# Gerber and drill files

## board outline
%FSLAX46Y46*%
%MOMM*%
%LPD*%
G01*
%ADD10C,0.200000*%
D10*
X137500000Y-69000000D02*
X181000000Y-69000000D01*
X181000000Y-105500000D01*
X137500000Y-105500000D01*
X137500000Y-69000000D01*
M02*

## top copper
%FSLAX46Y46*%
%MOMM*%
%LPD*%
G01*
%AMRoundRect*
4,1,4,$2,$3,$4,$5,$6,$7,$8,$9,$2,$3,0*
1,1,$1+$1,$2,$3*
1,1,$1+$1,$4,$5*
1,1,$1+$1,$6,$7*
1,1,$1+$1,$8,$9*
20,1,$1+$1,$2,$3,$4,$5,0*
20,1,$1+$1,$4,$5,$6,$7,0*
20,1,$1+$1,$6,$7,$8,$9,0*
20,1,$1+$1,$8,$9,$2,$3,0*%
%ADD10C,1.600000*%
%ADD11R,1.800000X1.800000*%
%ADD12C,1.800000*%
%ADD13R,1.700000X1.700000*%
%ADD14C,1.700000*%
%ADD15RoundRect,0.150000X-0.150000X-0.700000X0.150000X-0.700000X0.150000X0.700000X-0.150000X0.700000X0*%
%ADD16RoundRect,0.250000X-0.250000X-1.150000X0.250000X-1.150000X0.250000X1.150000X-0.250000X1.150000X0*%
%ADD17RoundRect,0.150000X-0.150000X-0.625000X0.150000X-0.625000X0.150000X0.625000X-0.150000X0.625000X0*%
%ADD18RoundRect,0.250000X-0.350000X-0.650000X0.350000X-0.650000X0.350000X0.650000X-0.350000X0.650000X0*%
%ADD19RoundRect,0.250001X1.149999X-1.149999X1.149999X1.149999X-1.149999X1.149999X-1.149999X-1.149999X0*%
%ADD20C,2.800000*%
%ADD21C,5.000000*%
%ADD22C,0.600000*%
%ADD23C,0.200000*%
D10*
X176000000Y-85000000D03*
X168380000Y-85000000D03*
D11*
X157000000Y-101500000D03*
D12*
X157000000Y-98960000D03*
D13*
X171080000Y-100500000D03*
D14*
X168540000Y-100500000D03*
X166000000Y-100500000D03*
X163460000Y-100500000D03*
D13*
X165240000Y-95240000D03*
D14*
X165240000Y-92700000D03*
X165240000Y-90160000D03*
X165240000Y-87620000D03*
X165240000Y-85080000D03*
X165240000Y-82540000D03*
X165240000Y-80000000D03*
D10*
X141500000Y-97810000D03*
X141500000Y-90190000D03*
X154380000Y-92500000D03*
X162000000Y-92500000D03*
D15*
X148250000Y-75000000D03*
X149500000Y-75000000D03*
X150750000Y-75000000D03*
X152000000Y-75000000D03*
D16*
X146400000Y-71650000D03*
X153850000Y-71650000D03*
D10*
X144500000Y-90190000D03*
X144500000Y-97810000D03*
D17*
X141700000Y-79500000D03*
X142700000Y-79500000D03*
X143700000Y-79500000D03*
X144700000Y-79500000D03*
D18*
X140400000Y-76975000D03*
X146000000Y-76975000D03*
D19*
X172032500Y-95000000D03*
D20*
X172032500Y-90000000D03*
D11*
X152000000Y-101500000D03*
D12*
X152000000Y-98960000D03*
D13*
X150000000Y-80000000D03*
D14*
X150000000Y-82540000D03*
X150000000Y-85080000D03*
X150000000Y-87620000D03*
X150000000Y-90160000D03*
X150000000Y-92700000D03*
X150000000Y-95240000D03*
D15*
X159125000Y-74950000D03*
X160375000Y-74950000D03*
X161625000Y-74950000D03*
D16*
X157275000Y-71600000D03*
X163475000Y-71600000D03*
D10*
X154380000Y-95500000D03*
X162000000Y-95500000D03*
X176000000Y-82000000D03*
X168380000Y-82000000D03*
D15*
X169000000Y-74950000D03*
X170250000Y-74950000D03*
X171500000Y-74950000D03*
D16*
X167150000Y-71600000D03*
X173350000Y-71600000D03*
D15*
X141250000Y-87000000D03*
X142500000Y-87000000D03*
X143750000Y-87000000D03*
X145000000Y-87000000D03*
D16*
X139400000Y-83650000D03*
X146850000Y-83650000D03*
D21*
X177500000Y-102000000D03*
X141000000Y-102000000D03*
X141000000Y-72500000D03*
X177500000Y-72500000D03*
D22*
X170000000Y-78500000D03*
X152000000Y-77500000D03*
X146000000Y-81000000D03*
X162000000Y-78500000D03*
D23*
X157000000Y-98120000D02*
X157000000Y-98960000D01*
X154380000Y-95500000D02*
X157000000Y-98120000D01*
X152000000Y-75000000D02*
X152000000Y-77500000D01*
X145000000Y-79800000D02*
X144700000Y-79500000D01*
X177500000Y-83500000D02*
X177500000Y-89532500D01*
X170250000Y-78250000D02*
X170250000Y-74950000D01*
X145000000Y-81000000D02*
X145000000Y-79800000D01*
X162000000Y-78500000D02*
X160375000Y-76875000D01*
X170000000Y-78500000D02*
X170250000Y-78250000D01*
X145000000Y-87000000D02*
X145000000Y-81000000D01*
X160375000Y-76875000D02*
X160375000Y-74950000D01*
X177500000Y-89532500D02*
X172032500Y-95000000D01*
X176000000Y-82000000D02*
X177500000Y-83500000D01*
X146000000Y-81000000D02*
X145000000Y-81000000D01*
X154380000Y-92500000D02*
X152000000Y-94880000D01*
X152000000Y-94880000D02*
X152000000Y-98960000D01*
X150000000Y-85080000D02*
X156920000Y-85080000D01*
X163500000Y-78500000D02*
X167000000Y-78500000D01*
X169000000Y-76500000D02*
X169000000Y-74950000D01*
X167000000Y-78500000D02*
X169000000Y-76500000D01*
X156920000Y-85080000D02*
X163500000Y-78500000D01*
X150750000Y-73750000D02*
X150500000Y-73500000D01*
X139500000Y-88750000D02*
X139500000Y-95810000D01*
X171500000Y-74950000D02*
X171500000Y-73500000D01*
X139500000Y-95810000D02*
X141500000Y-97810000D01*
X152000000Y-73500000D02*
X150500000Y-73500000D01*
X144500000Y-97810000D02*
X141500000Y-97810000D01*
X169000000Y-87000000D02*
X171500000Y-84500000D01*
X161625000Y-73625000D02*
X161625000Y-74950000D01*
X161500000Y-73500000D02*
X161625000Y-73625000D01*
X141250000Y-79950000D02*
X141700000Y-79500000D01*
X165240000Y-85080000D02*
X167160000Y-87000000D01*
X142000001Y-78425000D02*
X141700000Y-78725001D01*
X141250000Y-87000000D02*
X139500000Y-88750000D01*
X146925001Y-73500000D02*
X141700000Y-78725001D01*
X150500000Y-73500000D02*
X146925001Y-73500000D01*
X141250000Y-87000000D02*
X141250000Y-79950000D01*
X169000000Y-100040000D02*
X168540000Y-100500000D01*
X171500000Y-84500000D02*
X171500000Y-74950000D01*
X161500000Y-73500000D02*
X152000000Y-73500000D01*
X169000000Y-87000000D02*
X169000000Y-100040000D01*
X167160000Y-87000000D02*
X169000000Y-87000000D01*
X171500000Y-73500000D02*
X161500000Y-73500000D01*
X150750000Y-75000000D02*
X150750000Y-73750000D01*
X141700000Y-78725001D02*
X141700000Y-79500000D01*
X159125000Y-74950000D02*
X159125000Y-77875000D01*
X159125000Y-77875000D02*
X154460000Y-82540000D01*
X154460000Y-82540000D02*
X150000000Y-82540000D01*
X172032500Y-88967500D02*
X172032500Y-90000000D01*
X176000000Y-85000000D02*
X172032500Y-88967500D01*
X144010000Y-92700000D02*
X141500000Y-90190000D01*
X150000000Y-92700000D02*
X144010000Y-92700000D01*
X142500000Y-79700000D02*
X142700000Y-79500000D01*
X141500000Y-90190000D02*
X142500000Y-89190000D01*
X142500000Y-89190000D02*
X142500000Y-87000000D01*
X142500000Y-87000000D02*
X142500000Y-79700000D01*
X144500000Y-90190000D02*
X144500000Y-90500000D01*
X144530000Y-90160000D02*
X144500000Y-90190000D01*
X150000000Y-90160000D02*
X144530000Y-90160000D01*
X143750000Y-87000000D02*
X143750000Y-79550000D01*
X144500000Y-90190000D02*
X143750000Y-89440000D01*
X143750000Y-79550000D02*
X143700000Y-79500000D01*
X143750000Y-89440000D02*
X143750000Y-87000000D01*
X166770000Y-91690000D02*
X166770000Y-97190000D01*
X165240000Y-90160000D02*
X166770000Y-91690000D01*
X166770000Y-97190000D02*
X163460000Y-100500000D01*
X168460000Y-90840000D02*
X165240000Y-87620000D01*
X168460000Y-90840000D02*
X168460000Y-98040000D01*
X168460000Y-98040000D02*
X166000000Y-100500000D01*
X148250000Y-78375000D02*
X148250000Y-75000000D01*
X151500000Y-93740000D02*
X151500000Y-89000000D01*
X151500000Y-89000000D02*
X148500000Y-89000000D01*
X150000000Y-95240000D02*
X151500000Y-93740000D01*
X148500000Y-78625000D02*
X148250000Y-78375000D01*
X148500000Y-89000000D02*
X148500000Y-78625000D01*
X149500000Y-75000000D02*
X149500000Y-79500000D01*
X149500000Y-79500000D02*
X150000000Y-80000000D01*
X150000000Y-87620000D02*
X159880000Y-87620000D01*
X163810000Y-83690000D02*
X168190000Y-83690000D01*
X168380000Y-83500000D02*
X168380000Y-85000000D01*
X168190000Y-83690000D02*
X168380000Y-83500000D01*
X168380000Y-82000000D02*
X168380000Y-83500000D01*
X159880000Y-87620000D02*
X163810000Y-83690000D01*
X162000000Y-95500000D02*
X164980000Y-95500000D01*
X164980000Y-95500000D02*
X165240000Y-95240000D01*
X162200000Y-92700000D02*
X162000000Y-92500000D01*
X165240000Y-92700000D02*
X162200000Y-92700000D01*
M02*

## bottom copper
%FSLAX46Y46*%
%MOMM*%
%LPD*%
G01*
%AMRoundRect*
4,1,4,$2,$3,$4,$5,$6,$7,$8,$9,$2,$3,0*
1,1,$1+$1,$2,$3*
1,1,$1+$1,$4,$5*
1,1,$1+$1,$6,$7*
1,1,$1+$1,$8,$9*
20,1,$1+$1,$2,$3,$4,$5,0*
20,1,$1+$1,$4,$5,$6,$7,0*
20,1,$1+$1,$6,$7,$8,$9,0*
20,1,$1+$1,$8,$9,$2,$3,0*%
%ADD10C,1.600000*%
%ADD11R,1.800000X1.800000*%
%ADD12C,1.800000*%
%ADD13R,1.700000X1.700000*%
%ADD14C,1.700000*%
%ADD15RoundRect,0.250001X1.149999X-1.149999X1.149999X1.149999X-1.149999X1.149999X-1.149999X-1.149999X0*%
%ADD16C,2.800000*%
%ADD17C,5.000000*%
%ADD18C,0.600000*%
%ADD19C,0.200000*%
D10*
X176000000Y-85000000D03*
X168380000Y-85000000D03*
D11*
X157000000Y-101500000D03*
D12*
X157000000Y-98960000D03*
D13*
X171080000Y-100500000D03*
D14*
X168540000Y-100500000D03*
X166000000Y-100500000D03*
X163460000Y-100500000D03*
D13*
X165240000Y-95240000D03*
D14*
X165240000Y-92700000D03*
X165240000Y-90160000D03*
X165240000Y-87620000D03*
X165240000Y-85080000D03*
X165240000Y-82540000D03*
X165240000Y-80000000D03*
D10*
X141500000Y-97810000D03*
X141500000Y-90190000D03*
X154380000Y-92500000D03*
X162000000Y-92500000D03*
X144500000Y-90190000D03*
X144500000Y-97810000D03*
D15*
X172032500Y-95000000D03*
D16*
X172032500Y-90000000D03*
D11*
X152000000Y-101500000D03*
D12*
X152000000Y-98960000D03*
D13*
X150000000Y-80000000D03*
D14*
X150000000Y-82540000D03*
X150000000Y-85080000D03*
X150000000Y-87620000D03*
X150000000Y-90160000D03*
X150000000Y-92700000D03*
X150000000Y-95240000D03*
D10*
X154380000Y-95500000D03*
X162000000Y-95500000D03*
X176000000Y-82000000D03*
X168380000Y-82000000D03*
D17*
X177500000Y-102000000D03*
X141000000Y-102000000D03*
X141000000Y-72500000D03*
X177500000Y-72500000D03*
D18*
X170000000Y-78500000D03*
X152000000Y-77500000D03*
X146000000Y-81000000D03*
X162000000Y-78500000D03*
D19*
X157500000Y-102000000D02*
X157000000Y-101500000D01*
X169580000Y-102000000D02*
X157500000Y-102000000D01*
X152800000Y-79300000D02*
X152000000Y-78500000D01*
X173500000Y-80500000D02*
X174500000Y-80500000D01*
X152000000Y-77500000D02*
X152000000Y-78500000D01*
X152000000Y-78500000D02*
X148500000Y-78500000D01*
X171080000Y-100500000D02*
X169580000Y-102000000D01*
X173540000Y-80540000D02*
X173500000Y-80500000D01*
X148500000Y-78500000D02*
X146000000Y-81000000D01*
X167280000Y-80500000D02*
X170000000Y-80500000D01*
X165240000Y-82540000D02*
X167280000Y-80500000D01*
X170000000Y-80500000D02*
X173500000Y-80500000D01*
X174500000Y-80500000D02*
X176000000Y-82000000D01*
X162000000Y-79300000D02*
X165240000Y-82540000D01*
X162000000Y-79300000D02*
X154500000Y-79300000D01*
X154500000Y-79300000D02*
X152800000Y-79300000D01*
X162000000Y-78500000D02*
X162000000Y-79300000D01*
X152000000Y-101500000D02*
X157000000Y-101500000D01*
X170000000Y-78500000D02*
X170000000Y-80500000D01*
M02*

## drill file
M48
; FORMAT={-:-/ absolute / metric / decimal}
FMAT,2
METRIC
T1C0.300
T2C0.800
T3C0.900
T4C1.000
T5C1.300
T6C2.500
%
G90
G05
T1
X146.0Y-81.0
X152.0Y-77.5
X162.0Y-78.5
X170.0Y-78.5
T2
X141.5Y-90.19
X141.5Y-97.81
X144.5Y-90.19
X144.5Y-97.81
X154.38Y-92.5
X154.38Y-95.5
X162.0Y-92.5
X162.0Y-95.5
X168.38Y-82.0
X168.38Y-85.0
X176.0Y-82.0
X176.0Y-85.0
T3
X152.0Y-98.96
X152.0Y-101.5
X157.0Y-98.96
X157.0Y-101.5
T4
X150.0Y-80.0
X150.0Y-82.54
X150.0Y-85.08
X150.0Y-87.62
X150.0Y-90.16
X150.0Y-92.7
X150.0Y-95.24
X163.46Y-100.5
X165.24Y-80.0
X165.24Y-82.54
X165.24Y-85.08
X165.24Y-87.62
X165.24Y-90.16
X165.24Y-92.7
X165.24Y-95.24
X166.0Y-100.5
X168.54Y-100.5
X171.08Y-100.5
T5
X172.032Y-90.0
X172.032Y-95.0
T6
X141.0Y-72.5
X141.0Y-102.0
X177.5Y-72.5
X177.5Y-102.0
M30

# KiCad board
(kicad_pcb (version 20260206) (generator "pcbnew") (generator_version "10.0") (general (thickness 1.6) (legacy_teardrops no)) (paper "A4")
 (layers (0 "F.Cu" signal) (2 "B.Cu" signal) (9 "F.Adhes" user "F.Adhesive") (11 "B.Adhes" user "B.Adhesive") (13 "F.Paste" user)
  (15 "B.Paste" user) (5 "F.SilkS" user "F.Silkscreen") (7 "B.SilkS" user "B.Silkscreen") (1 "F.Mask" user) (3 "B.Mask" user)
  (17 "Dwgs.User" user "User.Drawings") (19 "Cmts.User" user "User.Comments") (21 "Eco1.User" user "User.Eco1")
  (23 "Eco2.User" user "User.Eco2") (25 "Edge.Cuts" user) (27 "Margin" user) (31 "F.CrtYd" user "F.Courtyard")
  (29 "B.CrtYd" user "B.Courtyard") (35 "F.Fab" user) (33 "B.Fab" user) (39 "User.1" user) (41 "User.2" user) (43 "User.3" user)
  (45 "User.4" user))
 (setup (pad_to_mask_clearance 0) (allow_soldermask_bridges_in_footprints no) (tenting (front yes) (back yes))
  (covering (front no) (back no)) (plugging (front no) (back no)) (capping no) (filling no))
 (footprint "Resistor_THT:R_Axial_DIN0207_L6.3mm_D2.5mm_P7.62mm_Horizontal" (layer "F.Cu") (at 176 85 180)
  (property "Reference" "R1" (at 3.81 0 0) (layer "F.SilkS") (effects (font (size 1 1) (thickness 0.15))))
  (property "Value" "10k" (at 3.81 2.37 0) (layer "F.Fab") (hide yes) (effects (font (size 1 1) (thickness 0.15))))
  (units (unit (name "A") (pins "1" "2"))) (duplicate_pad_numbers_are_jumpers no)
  (pad "1" thru_hole circle (at 0 0 180) (size 1.6 1.6) (drill 0.8) (layers "*.Cu" "*.Mask") (remove_unused_layers no)
   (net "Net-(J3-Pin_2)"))
  (pad "2" thru_hole circle (at 7.62 0 180) (size 1.6 1.6) (drill 0.8) (layers "*.Cu" "*.Mask") (remove_unused_layers no)
   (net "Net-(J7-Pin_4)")))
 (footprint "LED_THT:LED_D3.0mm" (layer "F.Cu") (at 157 101.5 90)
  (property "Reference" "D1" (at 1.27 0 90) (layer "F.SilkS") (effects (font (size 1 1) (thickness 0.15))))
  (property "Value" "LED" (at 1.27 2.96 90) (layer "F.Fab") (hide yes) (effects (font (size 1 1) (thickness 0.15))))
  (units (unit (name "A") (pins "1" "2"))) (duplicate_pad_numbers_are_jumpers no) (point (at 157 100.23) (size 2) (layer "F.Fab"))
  (pad "1" thru_hole rect (at 0 0 90) (size 1.8 1.8) (drill 0.9) (layers "*.Cu" "*.Mask") (remove_unused_layers no) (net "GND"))
  (pad "2" thru_hole circle (at 2.54 0 90) (size 1.8 1.8) (drill 0.9) (layers "*.Cu" "*.Mask") (remove_unused_layers no) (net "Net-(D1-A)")))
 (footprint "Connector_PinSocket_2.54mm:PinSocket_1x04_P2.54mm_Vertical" (layer "F.Cu") (at 171.08 100.5 -90)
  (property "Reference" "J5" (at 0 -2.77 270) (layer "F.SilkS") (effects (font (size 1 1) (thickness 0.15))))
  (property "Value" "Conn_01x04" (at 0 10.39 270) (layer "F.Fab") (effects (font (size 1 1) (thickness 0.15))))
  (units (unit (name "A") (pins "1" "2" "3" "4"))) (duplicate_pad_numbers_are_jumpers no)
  (pad "1" thru_hole rect (at 0 0 270) (size 1.7 1.7) (drill 1) (layers "*.Cu" "*.Mask") (remove_unused_layers no) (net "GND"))
  (pad "2" thru_hole circle (at 0 2.54 270) (size 1.7 1.7) (drill 1) (layers "*.Cu" "*.Mask") (remove_unused_layers no)
   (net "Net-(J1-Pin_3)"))
  (pad "3" thru_hole circle (at 0 5.08 270) (size 1.7 1.7) (drill 1) (layers "*.Cu" "*.Mask") (remove_unused_layers no)
   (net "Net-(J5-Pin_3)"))
  (pad "4" thru_hole circle (at 0 7.62 270) (size 1.7 1.7) (drill 1) (layers "*.Cu" "*.Mask") (remove_unused_layers no)
   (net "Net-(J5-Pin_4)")))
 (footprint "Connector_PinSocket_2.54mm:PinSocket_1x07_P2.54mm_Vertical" (layer "F.Cu") (at 165.24 95.24 180)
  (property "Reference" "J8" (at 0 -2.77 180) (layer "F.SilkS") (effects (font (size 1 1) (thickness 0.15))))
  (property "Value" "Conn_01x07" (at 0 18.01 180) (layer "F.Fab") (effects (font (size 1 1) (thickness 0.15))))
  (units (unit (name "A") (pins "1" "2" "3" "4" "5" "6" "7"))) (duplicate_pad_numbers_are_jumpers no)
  (pad "1" thru_hole rect (at 0 0 180) (size 1.7 1.7) (drill 1) (layers "*.Cu" "*.Mask") (remove_unused_layers no) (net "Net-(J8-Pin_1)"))
  (pad "2" thru_hole circle (at 0 2.54 180) (size 1.7 1.7) (drill 1) (layers "*.Cu" "*.Mask") (remove_unused_layers no)
   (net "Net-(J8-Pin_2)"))
  (pad "3" thru_hole circle (at 0 5.08 180) (size 1.7 1.7) (drill 1) (layers "*.Cu" "*.Mask") (remove_unused_layers no)
   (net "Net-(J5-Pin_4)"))
  (pad "4" thru_hole circle (at 0 7.62 180) (size 1.7 1.7) (drill 1) (layers "*.Cu" "*.Mask") (remove_unused_layers no)
   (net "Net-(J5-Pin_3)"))
  (pad "5" thru_hole circle (at 0 10.16 180) (size 1.7 1.7) (drill 1) (layers "*.Cu" "*.Mask") (remove_unused_layers no)
   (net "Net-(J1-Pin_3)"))
  (pad "6" thru_hole circle (at 0 12.7 180) (size 1.7 1.7) (drill 1) (layers "*.Cu" "*.Mask") (remove_unused_layers no) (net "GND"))
  (pad "7" thru_hole circle (at 0 15.24 180) (size 1.7 1.7) (drill 1) (layers "*.Cu" "*.Mask") (remove_unused_layers no)
   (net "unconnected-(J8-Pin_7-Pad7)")))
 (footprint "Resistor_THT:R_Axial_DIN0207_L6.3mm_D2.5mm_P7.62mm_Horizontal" (layer "F.Cu") (at 141.5 97.81 90)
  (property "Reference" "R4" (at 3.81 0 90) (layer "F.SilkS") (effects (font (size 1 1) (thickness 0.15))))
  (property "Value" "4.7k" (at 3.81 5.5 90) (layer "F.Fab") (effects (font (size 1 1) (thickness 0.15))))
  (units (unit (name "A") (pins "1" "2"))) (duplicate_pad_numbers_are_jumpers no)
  (pad "1" thru_hole circle (at 0 0 90) (size 1.6 1.6) (drill 0.8) (layers "*.Cu" "*.Mask") (remove_unused_layers no) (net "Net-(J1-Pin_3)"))
  (pad "2" thru_hole circle (at 7.62 0 90) (size 1.6 1.6) (drill 0.8) (layers "*.Cu" "*.Mask") (remove_unused_layers no)
   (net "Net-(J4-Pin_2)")))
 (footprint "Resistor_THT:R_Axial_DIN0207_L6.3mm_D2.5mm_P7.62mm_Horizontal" (layer "F.Cu") (at 154.38 92.5)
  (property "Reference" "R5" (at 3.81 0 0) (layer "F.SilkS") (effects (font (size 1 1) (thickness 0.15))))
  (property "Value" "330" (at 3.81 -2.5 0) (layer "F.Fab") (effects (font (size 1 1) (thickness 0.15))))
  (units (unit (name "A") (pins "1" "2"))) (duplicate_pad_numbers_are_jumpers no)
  (pad "1" thru_hole circle (at 0 0) (size 1.6 1.6) (drill 0.8) (layers "*.Cu" "*.Mask") (remove_unused_layers no) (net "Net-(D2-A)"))
  (pad "2" thru_hole circle (at 7.62 0) (size 1.6 1.6) (drill 0.8) (layers "*.Cu" "*.Mask") (remove_unused_layers no) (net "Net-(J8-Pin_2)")))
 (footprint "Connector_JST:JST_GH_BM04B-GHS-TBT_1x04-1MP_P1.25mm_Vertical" (layer "F.Cu") (at 150.125 73.05)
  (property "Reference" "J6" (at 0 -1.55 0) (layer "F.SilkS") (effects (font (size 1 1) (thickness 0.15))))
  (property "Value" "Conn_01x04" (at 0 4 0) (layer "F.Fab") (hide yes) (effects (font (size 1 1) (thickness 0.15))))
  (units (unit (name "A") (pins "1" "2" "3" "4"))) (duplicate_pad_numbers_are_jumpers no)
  (pad "1" smd roundrect (at -1.875 1.95) (size 0.6 1.7) (layers "F.Cu" "F.Mask" "F.Paste") (roundrect_rratio 0.25) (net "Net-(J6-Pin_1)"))
  (pad "2" smd roundrect (at -0.625 1.95) (size 0.6 1.7) (layers "F.Cu" "F.Mask" "F.Paste") (roundrect_rratio 0.25) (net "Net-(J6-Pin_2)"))
  (pad "3" smd roundrect (at 0.625 1.95) (size 0.6 1.7) (layers "F.Cu" "F.Mask" "F.Paste") (roundrect_rratio 0.25) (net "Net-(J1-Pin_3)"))
  (pad "4" smd roundrect (at 1.875 1.95) (size 0.6 1.7) (layers "F.Cu" "F.Mask" "F.Paste") (roundrect_rratio 0.25) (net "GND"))
  (pad "MP" smd roundrect (at -3.725 -1.4) (size 1 2.8) (layers "F.Cu" "F.Mask" "F.Paste") (roundrect_rratio 0.25))
  (pad "MP" smd roundrect (at 3.725 -1.4) (size 1 2.8) (layers "F.Cu" "F.Mask" "F.Paste") (roundrect_rratio 0.25)))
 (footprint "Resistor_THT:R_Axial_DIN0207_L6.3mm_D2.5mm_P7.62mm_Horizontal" (layer "F.Cu") (at 144.5 90.19 -90)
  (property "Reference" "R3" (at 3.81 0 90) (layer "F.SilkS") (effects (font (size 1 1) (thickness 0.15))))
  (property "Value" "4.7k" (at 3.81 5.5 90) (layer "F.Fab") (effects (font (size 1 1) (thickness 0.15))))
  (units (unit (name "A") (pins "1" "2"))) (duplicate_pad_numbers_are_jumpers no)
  (pad "1" thru_hole circle (at 0 0 270) (size 1.6 1.6) (drill 0.8) (layers "*.Cu" "*.Mask") (remove_unused_layers no)
   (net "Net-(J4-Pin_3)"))
  (pad "2" thru_hole circle (at 7.62 0 270) (size 1.6 1.6) (drill 0.8) (layers "*.Cu" "*.Mask") (remove_unused_layers no)
   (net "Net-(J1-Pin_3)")))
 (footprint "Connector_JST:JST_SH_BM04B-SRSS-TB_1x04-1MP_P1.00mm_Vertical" (layer "F.Cu") (at 143.2 78.175)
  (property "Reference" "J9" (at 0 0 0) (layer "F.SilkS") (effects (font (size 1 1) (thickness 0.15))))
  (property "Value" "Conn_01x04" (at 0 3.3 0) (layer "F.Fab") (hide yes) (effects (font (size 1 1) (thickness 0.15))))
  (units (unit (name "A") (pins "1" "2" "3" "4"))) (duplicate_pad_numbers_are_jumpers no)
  (pad "1" smd roundrect (at -1.5 1.325) (size 0.6 1.55) (layers "F.Cu" "F.Mask" "F.Paste") (roundrect_rratio 0.25) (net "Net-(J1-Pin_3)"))
  (pad "2" smd roundrect (at -0.5 1.325) (size 0.6 1.55) (layers "F.Cu" "F.Mask" "F.Paste") (roundrect_rratio 0.25) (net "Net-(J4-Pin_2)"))
  (pad "3" smd roundrect (at 0.5 1.325) (size 0.6 1.55) (layers "F.Cu" "F.Mask" "F.Paste") (roundrect_rratio 0.25) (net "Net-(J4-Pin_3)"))
  (pad "4" smd roundrect (at 1.5 1.325) (size 0.6 1.55) (layers "F.Cu" "F.Mask" "F.Paste") (roundrect_rratio 0.25) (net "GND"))
  (pad "MP" smd roundrect (at -2.8 -1.2) (size 1.2 1.8) (layers "F.Cu" "F.Mask" "F.Paste") (roundrect_rratio 0.208333))
  (pad "MP" smd roundrect (at 2.8 -1.2) (size 1.2 1.8) (layers "F.Cu" "F.Mask" "F.Paste") (roundrect_rratio 0.208333)))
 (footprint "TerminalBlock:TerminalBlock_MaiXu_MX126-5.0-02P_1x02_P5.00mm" (layer "F.Cu") (at 172.0325 95 90)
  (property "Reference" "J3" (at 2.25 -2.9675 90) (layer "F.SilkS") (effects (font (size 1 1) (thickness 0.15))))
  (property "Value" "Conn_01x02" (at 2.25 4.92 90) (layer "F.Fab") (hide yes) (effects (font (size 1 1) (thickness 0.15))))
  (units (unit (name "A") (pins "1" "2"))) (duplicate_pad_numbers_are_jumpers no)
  (pad "1" thru_hole roundrect (at 0 0 90) (size 2.8 2.8) (drill 1.3) (layers "*.Cu" "*.Mask") (remove_unused_layers no)
   (roundrect_rratio 0.089286) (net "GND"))
  (pad "2" thru_hole circle (at 5 0 90) (size 2.8 2.8) (drill 1.3) (layers "*.Cu" "*.Mask") (remove_unused_layers no) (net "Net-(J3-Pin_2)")))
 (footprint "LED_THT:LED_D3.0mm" (layer "F.Cu") (at 152 101.5 90)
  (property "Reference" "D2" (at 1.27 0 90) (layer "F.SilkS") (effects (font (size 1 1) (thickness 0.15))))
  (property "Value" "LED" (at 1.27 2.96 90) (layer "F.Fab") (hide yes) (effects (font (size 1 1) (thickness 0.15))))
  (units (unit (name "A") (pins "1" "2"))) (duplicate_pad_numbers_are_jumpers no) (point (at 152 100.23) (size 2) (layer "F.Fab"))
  (pad "1" thru_hole rect (at 0 0 90) (size 1.8 1.8) (drill 0.9) (layers "*.Cu" "*.Mask") (remove_unused_layers no) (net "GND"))
  (pad "2" thru_hole circle (at 2.54 0 90) (size 1.8 1.8) (drill 0.9) (layers "*.Cu" "*.Mask") (remove_unused_layers no) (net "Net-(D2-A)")))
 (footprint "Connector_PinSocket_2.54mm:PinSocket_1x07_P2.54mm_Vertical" (layer "F.Cu") (at 150 80)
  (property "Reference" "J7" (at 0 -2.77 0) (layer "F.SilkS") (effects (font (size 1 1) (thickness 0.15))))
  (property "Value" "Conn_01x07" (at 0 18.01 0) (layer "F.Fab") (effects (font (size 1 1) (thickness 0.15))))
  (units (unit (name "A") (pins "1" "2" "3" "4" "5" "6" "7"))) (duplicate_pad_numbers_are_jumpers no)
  (pad "1" thru_hole rect (at 0 0) (size 1.7 1.7) (drill 1) (layers "*.Cu" "*.Mask") (remove_unused_layers no) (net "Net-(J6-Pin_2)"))
  (pad "2" thru_hole circle (at 0 2.54) (size 1.7 1.7) (drill 1) (layers "*.Cu" "*.Mask") (remove_unused_layers no) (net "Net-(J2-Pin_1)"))
  (pad "3" thru_hole circle (at 0 5.08) (size 1.7 1.7) (drill 1) (layers "*.Cu" "*.Mask") (remove_unused_layers no) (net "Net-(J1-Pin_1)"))
  (pad "4" thru_hole circle (at 0 7.62) (size 1.7 1.7) (drill 1) (layers "*.Cu" "*.Mask") (remove_unused_layers no) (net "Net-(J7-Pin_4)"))
  (pad "5" thru_hole circle (at 0 10.16) (size 1.7 1.7) (drill 1) (layers "*.Cu" "*.Mask") (remove_unused_layers no) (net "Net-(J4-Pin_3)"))
  (pad "6" thru_hole circle (at 0 12.7) (size 1.7 1.7) (drill 1) (layers "*.Cu" "*.Mask") (remove_unused_layers no) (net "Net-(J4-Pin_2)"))
  (pad "7" thru_hole circle (at 0 15.24) (size 1.7 1.7) (drill 1) (layers "*.Cu" "*.Mask") (remove_unused_layers no) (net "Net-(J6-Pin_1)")))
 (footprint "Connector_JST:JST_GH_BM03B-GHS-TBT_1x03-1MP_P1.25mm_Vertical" (layer "F.Cu") (at 160.375 73)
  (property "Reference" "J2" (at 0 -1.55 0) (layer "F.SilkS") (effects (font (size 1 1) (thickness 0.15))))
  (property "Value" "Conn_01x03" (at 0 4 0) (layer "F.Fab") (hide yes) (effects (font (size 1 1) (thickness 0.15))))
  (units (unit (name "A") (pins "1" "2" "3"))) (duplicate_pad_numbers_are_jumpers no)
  (pad "1" smd roundrect (at -1.25 1.95) (size 0.6 1.7) (layers "F.Cu" "F.Mask" "F.Paste") (roundrect_rratio 0.25) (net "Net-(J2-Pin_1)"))
  (pad "2" smd roundrect (at 0 1.95) (size 0.6 1.7) (layers "F.Cu" "F.Mask" "F.Paste") (roundrect_rratio 0.25) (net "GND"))
  (pad "3" smd roundrect (at 1.25 1.95) (size 0.6 1.7) (layers "F.Cu" "F.Mask" "F.Paste") (roundrect_rratio 0.25) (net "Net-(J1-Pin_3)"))
  (pad "MP" smd roundrect (at -3.1 -1.4) (size 1 2.8) (layers "F.Cu" "F.Mask" "F.Paste") (roundrect_rratio 0.25))
  (pad "MP" smd roundrect (at 3.1 -1.4) (size 1 2.8) (layers "F.Cu" "F.Mask" "F.Paste") (roundrect_rratio 0.25)))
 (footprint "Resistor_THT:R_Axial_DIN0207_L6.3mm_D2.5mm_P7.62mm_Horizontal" (layer "F.Cu") (at 154.38 95.5)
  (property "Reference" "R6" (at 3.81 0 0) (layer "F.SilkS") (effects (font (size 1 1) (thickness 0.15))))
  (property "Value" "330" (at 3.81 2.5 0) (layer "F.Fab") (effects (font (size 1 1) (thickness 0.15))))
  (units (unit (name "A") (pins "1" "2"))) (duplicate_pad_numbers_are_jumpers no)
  (pad "1" thru_hole circle (at 0 0) (size 1.6 1.6) (drill 0.8) (layers "*.Cu" "*.Mask") (remove_unused_layers no) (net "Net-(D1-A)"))
  (pad "2" thru_hole circle (at 7.62 0) (size 1.6 1.6) (drill 0.8) (layers "*.Cu" "*.Mask") (remove_unused_layers no) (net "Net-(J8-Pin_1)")))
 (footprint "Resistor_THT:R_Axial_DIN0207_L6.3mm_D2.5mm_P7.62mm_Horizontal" (layer "F.Cu") (at 176 82 180)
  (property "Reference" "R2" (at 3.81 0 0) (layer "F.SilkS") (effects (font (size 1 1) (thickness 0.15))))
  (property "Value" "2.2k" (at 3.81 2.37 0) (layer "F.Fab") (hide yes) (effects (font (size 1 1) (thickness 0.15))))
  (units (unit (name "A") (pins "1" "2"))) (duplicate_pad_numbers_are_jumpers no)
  (pad "1" thru_hole circle (at 0 0 180) (size 1.6 1.6) (drill 0.8) (layers "*.Cu" "*.Mask") (remove_unused_layers no) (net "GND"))
  (pad "2" thru_hole circle (at 7.62 0 180) (size 1.6 1.6) (drill 0.8) (layers "*.Cu" "*.Mask") (remove_unused_layers no)
   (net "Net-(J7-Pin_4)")))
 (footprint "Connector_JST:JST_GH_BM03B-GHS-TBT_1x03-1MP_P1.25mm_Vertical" (layer "F.Cu") (at 170.25 73)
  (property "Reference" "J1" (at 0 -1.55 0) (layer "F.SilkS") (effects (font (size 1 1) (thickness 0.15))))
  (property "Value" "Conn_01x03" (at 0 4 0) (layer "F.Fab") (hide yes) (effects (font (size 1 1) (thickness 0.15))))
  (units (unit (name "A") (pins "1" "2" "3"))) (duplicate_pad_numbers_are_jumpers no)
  (pad "1" smd roundrect (at -1.25 1.95) (size 0.6 1.7) (layers "F.Cu" "F.Mask" "F.Paste") (roundrect_rratio 0.25) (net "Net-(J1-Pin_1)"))
  (pad "2" smd roundrect (at 0 1.95) (size 0.6 1.7) (layers "F.Cu" "F.Mask" "F.Paste") (roundrect_rratio 0.25) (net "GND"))
  (pad "3" smd roundrect (at 1.25 1.95) (size 0.6 1.7) (layers "F.Cu" "F.Mask" "F.Paste") (roundrect_rratio 0.25) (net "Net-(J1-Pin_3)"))
  (pad "MP" smd roundrect (at -3.1 -1.4) (size 1 2.8) (layers "F.Cu" "F.Mask" "F.Paste") (roundrect_rratio 0.25))
  (pad "MP" smd roundrect (at 3.1 -1.4) (size 1 2.8) (layers "F.Cu" "F.Mask" "F.Paste") (roundrect_rratio 0.25)))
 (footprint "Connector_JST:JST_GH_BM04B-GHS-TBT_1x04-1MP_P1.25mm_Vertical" (layer "F.Cu") (at 143.125 85.05)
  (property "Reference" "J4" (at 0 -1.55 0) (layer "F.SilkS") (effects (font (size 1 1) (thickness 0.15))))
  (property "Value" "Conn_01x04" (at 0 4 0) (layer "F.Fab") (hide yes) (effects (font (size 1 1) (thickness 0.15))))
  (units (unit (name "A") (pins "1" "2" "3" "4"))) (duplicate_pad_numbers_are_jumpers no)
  (pad "1" smd roundrect (at -1.875 1.95) (size 0.6 1.7) (layers "F.Cu" "F.Mask" "F.Paste") (roundrect_rratio 0.25) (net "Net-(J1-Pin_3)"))
  (pad "2" smd roundrect (at -0.625 1.95) (size 0.6 1.7) (layers "F.Cu" "F.Mask" "F.Paste") (roundrect_rratio 0.25) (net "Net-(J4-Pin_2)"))
  (pad "3" smd roundrect (at 0.625 1.95) (size 0.6 1.7) (layers "F.Cu" "F.Mask" "F.Paste") (roundrect_rratio 0.25) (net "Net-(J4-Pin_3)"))
  (pad "4" smd roundrect (at 1.875 1.95) (size 0.6 1.7) (layers "F.Cu" "F.Mask" "F.Paste") (roundrect_rratio 0.25) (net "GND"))
  (pad "MP" smd roundrect (at -3.725 -1.4) (size 1 2.8) (layers "F.Cu" "F.Mask" "F.Paste") (roundrect_rratio 0.25))
  (pad "MP" smd roundrect (at 3.725 -1.4) (size 1 2.8) (layers "F.Cu" "F.Mask" "F.Paste") (roundrect_rratio 0.25)))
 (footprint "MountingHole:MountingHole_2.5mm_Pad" (layer "B.Cu") (at 177.5 102 180)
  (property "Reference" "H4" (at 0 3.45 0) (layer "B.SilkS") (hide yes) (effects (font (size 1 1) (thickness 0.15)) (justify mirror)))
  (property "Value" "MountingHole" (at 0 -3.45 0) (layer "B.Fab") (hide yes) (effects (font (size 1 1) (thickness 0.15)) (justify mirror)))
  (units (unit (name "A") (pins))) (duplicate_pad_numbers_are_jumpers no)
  (pad "1" thru_hole circle (at 0 0 180) (size 5 5) (drill 2.5) (layers "*.Cu" "*.Mask") (remove_unused_layers no) (zone_connect 2)))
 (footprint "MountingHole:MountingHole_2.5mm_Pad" (layer "B.Cu") (at 141 102 180)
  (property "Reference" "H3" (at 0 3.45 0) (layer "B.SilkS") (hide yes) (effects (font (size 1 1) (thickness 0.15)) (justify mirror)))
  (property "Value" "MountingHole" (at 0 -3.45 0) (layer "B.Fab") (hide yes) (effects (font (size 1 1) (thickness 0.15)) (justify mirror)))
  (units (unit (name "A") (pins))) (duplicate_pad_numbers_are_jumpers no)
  (pad "1" thru_hole circle (at 0 0 180) (size 5 5) (drill 2.5) (layers "*.Cu" "*.Mask") (remove_unused_layers no) (zone_connect 2)))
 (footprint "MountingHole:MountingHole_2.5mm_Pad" (layer "B.Cu") (at 141 72.5 180)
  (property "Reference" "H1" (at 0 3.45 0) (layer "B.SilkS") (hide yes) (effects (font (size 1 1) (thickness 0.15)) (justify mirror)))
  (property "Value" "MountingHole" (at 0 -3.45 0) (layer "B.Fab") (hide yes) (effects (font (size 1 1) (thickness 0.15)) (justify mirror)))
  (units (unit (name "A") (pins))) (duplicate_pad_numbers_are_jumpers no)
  (pad "1" thru_hole circle (at 0 0 180) (size 5 5) (drill 2.5) (layers "*.Cu" "*.Mask") (remove_unused_layers no) (zone_connect 2)))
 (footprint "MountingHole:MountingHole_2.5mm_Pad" (layer "B.Cu") (at 177.5 72.5 180)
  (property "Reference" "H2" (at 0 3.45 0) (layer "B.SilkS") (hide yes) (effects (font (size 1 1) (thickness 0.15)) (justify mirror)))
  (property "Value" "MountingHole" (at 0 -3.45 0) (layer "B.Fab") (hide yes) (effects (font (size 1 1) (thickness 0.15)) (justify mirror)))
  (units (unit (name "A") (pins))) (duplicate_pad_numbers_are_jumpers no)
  (pad "1" thru_hole circle (at 0 0 180) (size 5 5) (drill 2.5) (layers "*.Cu" "*.Mask") (remove_unused_layers no) (zone_connect 2)))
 (gr_rect (start 137.5 69) (end 181 105.5) (stroke (width 0.2) (type solid)) (fill no) (layer "Edge.Cuts"))
 (segment (start 157 98.12) (end 157 98.96) (width 0.2) (layer "F.Cu") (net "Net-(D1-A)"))
 (segment (start 154.38 95.5) (end 157 98.12) (width 0.2) (layer "F.Cu") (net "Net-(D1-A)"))
 (segment (start 152 75) (end 152 77.5) (width 0.2) (layer "F.Cu") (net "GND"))
 (segment (start 145 79.8) (end 144.7 79.5) (width 0.2) (layer "F.Cu") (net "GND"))
 (segment (start 177.5 83.5) (end 177.5 89.5325) (width 0.2) (layer "F.Cu") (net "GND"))
 (segment (start 170.25 78.25) (end 170.25 74.95) (width 0.2) (layer "F.Cu") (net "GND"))
 (segment (start 145 81) (end 145 79.8) (width 0.2) (layer "F.Cu") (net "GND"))
 (segment (start 162 78.5) (end 160.375 76.875) (width 0.2) (layer "F.Cu") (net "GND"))
 (segment (start 170 78.5) (end 170.25 78.25) (width 0.2) (layer "F.Cu") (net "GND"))
 (segment (start 145 87) (end 145 81) (width 0.2) (layer "F.Cu") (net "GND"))
 (segment (start 160.375 76.875) (end 160.375 74.95) (width 0.2) (layer "F.Cu") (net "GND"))
 (segment (start 177.5 89.5325) (end 172.0325 95) (width 0.2) (layer "F.Cu") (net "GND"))
 (segment (start 176 82) (end 177.5 83.5) (width 0.2) (layer "F.Cu") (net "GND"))
 (segment (start 146 81) (end 145 81) (width 0.2) (layer "F.Cu") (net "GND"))
 (via (at 170 78.5) (size 0.6) (drill 0.3) (layers "F.Cu" "B.Cu") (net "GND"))
 (via (at 152 77.5) (size 0.6) (drill 0.3) (layers "F.Cu" "B.Cu") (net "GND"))
 (via (at 146 81) (size 0.6) (drill 0.3) (layers "F.Cu" "B.Cu") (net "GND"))
 (via (at 162 78.5) (size 0.6) (drill 0.3) (layers "F.Cu" "B.Cu") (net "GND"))
 (segment (start 157.5 102) (end 157 101.5) (width 0.2) (layer "B.Cu") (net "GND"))
 (segment (start 169.58 102) (end 157.5 102) (width 0.2) (layer "B.Cu") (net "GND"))
 (segment (start 152.8 79.3) (end 152 78.5) (width 0.2) (layer "B.Cu") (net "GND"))
 (segment (start 173.5 80.5) (end 174.5 80.5) (width 0.2) (layer "B.Cu") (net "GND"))
 (segment (start 152 77.5) (end 152 78.5) (width 0.2) (layer "B.Cu") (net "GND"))
 (segment (start 152 78.5) (end 148.5 78.5) (width 0.2) (layer "B.Cu") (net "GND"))
 (segment (start 171.08 100.5) (end 169.58 102) (width 0.2) (layer "B.Cu") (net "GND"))
 (segment (start 173.54 80.54) (end 173.5 80.5) (width 0.2) (layer "B.Cu") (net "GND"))
 (segment (start 148.5 78.5) (end 146 81) (width 0.2) (layer "B.Cu") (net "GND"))
 (segment (start 167.28 80.5) (end 170 80.5) (width 0.2) (layer "B.Cu") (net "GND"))
 (segment (start 165.24 82.54) (end 167.28 80.5) (width 0.2) (layer "B.Cu") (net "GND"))
 (segment (start 170 80.5) (end 173.5 80.5) (width 0.2) (layer "B.Cu") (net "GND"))
 (segment (start 174.5 80.5) (end 176 82) (width 0.2) (layer "B.Cu") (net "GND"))
 (segment (start 162 79.3) (end 165.24 82.54) (width 0.2) (layer "B.Cu") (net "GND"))
 (segment (start 162 79.3) (end 154.5 79.3) (width 0.2) (layer "B.Cu") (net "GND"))
 (segment (start 154.5 79.3) (end 152.8 79.3) (width 0.2) (layer "B.Cu") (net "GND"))
 (segment (start 162 78.5) (end 162 79.3) (width 0.2) (layer "B.Cu") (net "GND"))
 (segment (start 152 101.5) (end 157 101.5) (width 0.2) (layer "B.Cu") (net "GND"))
 (segment (start 170 78.5) (end 170 80.5) (width 0.2) (layer "B.Cu") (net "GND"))
 (segment (start 154.38 92.5) (end 152 94.88) (width 0.2) (layer "F.Cu") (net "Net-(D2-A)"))
 (segment (start 152 94.88) (end 152 98.96) (width 0.2) (layer "F.Cu") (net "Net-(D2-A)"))
 (segment (start 150 85.08) (end 156.92 85.08) (width 0.2) (layer "F.Cu") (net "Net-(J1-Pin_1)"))
 (segment (start 163.5 78.5) (end 167 78.5) (width 0.2) (layer "F.Cu") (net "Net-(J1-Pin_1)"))
 (segment (start 169 76.5) (end 169 74.95) (width 0.2) (layer "F.Cu") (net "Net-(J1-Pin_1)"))
 (segment (start 167 78.5) (end 169 76.5) (width 0.2) (layer "F.Cu") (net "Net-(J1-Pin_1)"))
 (segment (start 156.92 85.08) (end 163.5 78.5) (width 0.2) (layer "F.Cu") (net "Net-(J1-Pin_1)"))
 (segment (start 150.75 73.75) (end 150.5 73.5) (width 0.2) (layer "F.Cu") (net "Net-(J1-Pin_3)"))
 (segment (start 139.5 88.75) (end 139.5 95.81) (width 0.2) (layer "F.Cu") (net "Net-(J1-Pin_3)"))
 (segment (start 171.5 74.95) (end 171.5 73.5) (width 0.2) (layer "F.Cu") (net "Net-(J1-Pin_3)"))
 (segment (start 139.5 95.81) (end 141.5 97.81) (width 0.2) (layer "F.Cu") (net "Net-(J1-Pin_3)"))
 (segment (start 152 73.5) (end 150.5 73.5) (width 0.2) (layer "F.Cu") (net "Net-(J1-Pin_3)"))
 (segment (start 144.5 97.81) (end 141.5 97.81) (width 0.2) (layer "F.Cu") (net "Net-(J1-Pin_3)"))
 (segment (start 169 87) (end 171.5 84.5) (width 0.2) (layer "F.Cu") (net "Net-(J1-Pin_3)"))
 (segment (start 161.625 73.625) (end 161.625 74.95) (width 0.2) (layer "F.Cu") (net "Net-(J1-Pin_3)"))
 (segment (start 161.5 73.5) (end 161.625 73.625) (width 0.2) (layer "F.Cu") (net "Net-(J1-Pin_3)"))
 (segment (start 141.25 79.95) (end 141.7 79.5) (width 0.2) (layer "F.Cu") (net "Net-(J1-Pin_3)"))
 (segment (start 165.24 85.08) (end 167.16 87) (width 0.2) (layer "F.Cu") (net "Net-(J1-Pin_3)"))
 (segment (start 142.000001 78.425) (end 141.7 78.725001) (width 0.2) (layer "F.Cu") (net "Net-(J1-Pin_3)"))
 (segment (start 141.25 87) (end 139.5 88.75) (width 0.2) (layer "F.Cu") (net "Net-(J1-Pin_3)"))
 (segment (start 146.925001 73.5) (end 141.7 78.725001) (width 0.2) (layer "F.Cu") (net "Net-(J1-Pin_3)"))
 (segment (start 150.5 73.5) (end 146.925001 73.5) (width 0.2) (layer "F.Cu") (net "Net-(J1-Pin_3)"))
 (segment (start 141.25 87) (end 141.25 79.95) (width 0.2) (layer "F.Cu") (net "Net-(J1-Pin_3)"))
 (segment (start 169 100.04) (end 168.54 100.5) (width 0.2) (layer "F.Cu") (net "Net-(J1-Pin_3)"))
 (segment (start 171.5 84.5) (end 171.5 74.95) (width 0.2) (layer "F.Cu") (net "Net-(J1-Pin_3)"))
 (segment (start 161.5 73.5) (end 152 73.5) (width 0.2) (layer "F.Cu") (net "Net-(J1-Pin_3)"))
 (segment (start 169 87) (end 169 100.04) (width 0.2) (layer "F.Cu") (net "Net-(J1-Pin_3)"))
 (segment (start 167.16 87) (end 169 87) (width 0.2) (layer "F.Cu") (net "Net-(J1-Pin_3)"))
 (segment (start 171.5 73.5) (end 161.5 73.5) (width 0.2) (layer "F.Cu") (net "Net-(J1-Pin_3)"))
 (segment (start 150.75 75) (end 150.75 73.75) (width 0.2) (layer "F.Cu") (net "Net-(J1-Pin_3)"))
 (segment (start 141.7 78.725001) (end 141.7 79.5) (width 0.2) (layer "F.Cu") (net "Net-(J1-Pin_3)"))
 (segment (start 159.125 74.95) (end 159.125 77.875) (width 0.2) (layer "F.Cu") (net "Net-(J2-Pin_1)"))
 (segment (start 159.125 77.875) (end 154.46 82.54) (width 0.2) (layer "F.Cu") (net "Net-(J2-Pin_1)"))
 (segment (start 154.46 82.54) (end 150 82.54) (width 0.2) (layer "F.Cu") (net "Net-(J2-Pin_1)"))
 (segment (start 172.0325 88.9675) (end 172.0325 90) (width 0.2) (layer "F.Cu") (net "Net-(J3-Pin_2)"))
 (segment (start 176 85) (end 172.0325 88.9675) (width 0.2) (layer "F.Cu") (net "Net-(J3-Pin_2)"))
 (segment (start 144.01 92.7) (end 141.5 90.19) (width 0.2) (layer "F.Cu") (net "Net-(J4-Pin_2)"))
 (segment (start 150 92.7) (end 144.01 92.7) (width 0.2) (layer "F.Cu") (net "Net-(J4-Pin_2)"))
 (segment (start 142.5 79.7) (end 142.7 79.5) (width 0.2) (layer "F.Cu") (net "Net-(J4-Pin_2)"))
 (segment (start 141.5 90.19) (end 142.5 89.19) (width 0.2) (layer "F.Cu") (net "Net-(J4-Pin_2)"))
 (segment (start 142.5 89.19) (end 142.5 87) (width 0.2) (layer "F.Cu") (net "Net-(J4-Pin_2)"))
 (segment (start 142.5 87) (end 142.5 79.7) (width 0.2) (layer "F.Cu") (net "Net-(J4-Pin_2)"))
 (segment (start 144.5 90.19) (end 144.5 90.5) (width 0.2) (layer "F.Cu") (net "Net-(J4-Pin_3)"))
 (segment (start 144.53 90.16) (end 144.5 90.19) (width 0.2) (layer "F.Cu") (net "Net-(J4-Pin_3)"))
 (segment (start 150 90.16) (end 144.53 90.16) (width 0.2) (layer "F.Cu") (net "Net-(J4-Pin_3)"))
 (segment (start 143.75 87) (end 143.75 79.55) (width 0.2) (layer "F.Cu") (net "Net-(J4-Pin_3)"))
 (segment (start 144.5 90.19) (end 143.75 89.44) (width 0.2) (layer "F.Cu") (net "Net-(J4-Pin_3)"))
 (segment (start 143.75 79.55) (end 143.7 79.5) (width 0.2) (layer "F.Cu") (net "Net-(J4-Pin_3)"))
 (segment (start 143.75 89.44) (end 143.75 87) (width 0.2) (layer "F.Cu") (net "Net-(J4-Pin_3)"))
 (segment (start 166.77 91.69) (end 166.77 97.19) (width 0.2) (layer "F.Cu") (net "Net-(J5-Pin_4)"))
 (segment (start 165.24 90.16) (end 166.77 91.69) (width 0.2) (layer "F.Cu") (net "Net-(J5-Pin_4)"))
 (segment (start 166.77 97.19) (end 163.46 100.5) (width 0.2) (layer "F.Cu") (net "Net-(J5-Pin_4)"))
 (segment (start 168.46 90.84) (end 165.24 87.62) (width 0.2) (layer "F.Cu") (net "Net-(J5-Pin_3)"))
 (segment (start 168.46 90.84) (end 168.46 98.04) (width 0.2) (layer "F.Cu") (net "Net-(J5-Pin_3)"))
 (segment (start 168.46 98.04) (end 166 100.5) (width 0.2) (layer "F.Cu") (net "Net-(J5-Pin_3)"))
 (segment (start 148.25 78.375) (end 148.25 75) (width 0.2) (layer "F.Cu") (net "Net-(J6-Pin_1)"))
 (segment (start 151.5 93.74) (end 151.5 89) (width 0.2) (layer "F.Cu") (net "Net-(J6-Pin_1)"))
 (segment (start 151.5 89) (end 148.5 89) (width 0.2) (layer "F.Cu") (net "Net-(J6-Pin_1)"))
 (segment (start 150 95.24) (end 151.5 93.74) (width 0.2) (layer "F.Cu") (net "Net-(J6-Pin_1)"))
 (segment (start 148.5 78.625) (end 148.25 78.375) (width 0.2) (layer "F.Cu") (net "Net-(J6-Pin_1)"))
 (segment (start 148.5 89) (end 148.5 78.625) (width 0.2) (layer "F.Cu") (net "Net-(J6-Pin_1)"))
 (segment (start 149.5 75) (end 149.5 79.5) (width 0.2) (layer "F.Cu") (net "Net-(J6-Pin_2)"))
 (segment (start 149.5 79.5) (end 150 80) (width 0.2) (layer "F.Cu") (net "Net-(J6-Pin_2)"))
 (segment (start 150 87.62) (end 159.88 87.62) (width 0.2) (layer "F.Cu") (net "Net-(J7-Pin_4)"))
 (segment (start 163.81 83.69) (end 168.19 83.69) (width 0.2) (layer "F.Cu") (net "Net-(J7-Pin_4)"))
 (segment (start 168.38 83.5) (end 168.38 85) (width 0.2) (layer "F.Cu") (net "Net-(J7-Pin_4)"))
 (segment (start 168.19 83.69) (end 168.38 83.5) (width 0.2) (layer "F.Cu") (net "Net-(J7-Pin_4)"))
 (segment (start 168.38 82) (end 168.38 83.5) (width 0.2) (layer "F.Cu") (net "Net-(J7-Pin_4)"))
 (segment (start 159.88 87.62) (end 163.81 83.69) (width 0.2) (layer "F.Cu") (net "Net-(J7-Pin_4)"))
 (segment (start 162 95.5) (end 164.98 95.5) (width 0.2) (layer "F.Cu") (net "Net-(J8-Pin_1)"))
 (segment (start 164.98 95.5) (end 165.24 95.24) (width 0.2) (layer "F.Cu") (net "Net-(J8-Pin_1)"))
 (segment (start 162.2 92.7) (end 162 92.5) (width 0.2) (layer "F.Cu") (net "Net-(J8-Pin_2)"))
 (segment (start 165.24 92.7) (end 162.2 92.7) (width 0.2) (layer "F.Cu") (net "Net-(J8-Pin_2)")))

